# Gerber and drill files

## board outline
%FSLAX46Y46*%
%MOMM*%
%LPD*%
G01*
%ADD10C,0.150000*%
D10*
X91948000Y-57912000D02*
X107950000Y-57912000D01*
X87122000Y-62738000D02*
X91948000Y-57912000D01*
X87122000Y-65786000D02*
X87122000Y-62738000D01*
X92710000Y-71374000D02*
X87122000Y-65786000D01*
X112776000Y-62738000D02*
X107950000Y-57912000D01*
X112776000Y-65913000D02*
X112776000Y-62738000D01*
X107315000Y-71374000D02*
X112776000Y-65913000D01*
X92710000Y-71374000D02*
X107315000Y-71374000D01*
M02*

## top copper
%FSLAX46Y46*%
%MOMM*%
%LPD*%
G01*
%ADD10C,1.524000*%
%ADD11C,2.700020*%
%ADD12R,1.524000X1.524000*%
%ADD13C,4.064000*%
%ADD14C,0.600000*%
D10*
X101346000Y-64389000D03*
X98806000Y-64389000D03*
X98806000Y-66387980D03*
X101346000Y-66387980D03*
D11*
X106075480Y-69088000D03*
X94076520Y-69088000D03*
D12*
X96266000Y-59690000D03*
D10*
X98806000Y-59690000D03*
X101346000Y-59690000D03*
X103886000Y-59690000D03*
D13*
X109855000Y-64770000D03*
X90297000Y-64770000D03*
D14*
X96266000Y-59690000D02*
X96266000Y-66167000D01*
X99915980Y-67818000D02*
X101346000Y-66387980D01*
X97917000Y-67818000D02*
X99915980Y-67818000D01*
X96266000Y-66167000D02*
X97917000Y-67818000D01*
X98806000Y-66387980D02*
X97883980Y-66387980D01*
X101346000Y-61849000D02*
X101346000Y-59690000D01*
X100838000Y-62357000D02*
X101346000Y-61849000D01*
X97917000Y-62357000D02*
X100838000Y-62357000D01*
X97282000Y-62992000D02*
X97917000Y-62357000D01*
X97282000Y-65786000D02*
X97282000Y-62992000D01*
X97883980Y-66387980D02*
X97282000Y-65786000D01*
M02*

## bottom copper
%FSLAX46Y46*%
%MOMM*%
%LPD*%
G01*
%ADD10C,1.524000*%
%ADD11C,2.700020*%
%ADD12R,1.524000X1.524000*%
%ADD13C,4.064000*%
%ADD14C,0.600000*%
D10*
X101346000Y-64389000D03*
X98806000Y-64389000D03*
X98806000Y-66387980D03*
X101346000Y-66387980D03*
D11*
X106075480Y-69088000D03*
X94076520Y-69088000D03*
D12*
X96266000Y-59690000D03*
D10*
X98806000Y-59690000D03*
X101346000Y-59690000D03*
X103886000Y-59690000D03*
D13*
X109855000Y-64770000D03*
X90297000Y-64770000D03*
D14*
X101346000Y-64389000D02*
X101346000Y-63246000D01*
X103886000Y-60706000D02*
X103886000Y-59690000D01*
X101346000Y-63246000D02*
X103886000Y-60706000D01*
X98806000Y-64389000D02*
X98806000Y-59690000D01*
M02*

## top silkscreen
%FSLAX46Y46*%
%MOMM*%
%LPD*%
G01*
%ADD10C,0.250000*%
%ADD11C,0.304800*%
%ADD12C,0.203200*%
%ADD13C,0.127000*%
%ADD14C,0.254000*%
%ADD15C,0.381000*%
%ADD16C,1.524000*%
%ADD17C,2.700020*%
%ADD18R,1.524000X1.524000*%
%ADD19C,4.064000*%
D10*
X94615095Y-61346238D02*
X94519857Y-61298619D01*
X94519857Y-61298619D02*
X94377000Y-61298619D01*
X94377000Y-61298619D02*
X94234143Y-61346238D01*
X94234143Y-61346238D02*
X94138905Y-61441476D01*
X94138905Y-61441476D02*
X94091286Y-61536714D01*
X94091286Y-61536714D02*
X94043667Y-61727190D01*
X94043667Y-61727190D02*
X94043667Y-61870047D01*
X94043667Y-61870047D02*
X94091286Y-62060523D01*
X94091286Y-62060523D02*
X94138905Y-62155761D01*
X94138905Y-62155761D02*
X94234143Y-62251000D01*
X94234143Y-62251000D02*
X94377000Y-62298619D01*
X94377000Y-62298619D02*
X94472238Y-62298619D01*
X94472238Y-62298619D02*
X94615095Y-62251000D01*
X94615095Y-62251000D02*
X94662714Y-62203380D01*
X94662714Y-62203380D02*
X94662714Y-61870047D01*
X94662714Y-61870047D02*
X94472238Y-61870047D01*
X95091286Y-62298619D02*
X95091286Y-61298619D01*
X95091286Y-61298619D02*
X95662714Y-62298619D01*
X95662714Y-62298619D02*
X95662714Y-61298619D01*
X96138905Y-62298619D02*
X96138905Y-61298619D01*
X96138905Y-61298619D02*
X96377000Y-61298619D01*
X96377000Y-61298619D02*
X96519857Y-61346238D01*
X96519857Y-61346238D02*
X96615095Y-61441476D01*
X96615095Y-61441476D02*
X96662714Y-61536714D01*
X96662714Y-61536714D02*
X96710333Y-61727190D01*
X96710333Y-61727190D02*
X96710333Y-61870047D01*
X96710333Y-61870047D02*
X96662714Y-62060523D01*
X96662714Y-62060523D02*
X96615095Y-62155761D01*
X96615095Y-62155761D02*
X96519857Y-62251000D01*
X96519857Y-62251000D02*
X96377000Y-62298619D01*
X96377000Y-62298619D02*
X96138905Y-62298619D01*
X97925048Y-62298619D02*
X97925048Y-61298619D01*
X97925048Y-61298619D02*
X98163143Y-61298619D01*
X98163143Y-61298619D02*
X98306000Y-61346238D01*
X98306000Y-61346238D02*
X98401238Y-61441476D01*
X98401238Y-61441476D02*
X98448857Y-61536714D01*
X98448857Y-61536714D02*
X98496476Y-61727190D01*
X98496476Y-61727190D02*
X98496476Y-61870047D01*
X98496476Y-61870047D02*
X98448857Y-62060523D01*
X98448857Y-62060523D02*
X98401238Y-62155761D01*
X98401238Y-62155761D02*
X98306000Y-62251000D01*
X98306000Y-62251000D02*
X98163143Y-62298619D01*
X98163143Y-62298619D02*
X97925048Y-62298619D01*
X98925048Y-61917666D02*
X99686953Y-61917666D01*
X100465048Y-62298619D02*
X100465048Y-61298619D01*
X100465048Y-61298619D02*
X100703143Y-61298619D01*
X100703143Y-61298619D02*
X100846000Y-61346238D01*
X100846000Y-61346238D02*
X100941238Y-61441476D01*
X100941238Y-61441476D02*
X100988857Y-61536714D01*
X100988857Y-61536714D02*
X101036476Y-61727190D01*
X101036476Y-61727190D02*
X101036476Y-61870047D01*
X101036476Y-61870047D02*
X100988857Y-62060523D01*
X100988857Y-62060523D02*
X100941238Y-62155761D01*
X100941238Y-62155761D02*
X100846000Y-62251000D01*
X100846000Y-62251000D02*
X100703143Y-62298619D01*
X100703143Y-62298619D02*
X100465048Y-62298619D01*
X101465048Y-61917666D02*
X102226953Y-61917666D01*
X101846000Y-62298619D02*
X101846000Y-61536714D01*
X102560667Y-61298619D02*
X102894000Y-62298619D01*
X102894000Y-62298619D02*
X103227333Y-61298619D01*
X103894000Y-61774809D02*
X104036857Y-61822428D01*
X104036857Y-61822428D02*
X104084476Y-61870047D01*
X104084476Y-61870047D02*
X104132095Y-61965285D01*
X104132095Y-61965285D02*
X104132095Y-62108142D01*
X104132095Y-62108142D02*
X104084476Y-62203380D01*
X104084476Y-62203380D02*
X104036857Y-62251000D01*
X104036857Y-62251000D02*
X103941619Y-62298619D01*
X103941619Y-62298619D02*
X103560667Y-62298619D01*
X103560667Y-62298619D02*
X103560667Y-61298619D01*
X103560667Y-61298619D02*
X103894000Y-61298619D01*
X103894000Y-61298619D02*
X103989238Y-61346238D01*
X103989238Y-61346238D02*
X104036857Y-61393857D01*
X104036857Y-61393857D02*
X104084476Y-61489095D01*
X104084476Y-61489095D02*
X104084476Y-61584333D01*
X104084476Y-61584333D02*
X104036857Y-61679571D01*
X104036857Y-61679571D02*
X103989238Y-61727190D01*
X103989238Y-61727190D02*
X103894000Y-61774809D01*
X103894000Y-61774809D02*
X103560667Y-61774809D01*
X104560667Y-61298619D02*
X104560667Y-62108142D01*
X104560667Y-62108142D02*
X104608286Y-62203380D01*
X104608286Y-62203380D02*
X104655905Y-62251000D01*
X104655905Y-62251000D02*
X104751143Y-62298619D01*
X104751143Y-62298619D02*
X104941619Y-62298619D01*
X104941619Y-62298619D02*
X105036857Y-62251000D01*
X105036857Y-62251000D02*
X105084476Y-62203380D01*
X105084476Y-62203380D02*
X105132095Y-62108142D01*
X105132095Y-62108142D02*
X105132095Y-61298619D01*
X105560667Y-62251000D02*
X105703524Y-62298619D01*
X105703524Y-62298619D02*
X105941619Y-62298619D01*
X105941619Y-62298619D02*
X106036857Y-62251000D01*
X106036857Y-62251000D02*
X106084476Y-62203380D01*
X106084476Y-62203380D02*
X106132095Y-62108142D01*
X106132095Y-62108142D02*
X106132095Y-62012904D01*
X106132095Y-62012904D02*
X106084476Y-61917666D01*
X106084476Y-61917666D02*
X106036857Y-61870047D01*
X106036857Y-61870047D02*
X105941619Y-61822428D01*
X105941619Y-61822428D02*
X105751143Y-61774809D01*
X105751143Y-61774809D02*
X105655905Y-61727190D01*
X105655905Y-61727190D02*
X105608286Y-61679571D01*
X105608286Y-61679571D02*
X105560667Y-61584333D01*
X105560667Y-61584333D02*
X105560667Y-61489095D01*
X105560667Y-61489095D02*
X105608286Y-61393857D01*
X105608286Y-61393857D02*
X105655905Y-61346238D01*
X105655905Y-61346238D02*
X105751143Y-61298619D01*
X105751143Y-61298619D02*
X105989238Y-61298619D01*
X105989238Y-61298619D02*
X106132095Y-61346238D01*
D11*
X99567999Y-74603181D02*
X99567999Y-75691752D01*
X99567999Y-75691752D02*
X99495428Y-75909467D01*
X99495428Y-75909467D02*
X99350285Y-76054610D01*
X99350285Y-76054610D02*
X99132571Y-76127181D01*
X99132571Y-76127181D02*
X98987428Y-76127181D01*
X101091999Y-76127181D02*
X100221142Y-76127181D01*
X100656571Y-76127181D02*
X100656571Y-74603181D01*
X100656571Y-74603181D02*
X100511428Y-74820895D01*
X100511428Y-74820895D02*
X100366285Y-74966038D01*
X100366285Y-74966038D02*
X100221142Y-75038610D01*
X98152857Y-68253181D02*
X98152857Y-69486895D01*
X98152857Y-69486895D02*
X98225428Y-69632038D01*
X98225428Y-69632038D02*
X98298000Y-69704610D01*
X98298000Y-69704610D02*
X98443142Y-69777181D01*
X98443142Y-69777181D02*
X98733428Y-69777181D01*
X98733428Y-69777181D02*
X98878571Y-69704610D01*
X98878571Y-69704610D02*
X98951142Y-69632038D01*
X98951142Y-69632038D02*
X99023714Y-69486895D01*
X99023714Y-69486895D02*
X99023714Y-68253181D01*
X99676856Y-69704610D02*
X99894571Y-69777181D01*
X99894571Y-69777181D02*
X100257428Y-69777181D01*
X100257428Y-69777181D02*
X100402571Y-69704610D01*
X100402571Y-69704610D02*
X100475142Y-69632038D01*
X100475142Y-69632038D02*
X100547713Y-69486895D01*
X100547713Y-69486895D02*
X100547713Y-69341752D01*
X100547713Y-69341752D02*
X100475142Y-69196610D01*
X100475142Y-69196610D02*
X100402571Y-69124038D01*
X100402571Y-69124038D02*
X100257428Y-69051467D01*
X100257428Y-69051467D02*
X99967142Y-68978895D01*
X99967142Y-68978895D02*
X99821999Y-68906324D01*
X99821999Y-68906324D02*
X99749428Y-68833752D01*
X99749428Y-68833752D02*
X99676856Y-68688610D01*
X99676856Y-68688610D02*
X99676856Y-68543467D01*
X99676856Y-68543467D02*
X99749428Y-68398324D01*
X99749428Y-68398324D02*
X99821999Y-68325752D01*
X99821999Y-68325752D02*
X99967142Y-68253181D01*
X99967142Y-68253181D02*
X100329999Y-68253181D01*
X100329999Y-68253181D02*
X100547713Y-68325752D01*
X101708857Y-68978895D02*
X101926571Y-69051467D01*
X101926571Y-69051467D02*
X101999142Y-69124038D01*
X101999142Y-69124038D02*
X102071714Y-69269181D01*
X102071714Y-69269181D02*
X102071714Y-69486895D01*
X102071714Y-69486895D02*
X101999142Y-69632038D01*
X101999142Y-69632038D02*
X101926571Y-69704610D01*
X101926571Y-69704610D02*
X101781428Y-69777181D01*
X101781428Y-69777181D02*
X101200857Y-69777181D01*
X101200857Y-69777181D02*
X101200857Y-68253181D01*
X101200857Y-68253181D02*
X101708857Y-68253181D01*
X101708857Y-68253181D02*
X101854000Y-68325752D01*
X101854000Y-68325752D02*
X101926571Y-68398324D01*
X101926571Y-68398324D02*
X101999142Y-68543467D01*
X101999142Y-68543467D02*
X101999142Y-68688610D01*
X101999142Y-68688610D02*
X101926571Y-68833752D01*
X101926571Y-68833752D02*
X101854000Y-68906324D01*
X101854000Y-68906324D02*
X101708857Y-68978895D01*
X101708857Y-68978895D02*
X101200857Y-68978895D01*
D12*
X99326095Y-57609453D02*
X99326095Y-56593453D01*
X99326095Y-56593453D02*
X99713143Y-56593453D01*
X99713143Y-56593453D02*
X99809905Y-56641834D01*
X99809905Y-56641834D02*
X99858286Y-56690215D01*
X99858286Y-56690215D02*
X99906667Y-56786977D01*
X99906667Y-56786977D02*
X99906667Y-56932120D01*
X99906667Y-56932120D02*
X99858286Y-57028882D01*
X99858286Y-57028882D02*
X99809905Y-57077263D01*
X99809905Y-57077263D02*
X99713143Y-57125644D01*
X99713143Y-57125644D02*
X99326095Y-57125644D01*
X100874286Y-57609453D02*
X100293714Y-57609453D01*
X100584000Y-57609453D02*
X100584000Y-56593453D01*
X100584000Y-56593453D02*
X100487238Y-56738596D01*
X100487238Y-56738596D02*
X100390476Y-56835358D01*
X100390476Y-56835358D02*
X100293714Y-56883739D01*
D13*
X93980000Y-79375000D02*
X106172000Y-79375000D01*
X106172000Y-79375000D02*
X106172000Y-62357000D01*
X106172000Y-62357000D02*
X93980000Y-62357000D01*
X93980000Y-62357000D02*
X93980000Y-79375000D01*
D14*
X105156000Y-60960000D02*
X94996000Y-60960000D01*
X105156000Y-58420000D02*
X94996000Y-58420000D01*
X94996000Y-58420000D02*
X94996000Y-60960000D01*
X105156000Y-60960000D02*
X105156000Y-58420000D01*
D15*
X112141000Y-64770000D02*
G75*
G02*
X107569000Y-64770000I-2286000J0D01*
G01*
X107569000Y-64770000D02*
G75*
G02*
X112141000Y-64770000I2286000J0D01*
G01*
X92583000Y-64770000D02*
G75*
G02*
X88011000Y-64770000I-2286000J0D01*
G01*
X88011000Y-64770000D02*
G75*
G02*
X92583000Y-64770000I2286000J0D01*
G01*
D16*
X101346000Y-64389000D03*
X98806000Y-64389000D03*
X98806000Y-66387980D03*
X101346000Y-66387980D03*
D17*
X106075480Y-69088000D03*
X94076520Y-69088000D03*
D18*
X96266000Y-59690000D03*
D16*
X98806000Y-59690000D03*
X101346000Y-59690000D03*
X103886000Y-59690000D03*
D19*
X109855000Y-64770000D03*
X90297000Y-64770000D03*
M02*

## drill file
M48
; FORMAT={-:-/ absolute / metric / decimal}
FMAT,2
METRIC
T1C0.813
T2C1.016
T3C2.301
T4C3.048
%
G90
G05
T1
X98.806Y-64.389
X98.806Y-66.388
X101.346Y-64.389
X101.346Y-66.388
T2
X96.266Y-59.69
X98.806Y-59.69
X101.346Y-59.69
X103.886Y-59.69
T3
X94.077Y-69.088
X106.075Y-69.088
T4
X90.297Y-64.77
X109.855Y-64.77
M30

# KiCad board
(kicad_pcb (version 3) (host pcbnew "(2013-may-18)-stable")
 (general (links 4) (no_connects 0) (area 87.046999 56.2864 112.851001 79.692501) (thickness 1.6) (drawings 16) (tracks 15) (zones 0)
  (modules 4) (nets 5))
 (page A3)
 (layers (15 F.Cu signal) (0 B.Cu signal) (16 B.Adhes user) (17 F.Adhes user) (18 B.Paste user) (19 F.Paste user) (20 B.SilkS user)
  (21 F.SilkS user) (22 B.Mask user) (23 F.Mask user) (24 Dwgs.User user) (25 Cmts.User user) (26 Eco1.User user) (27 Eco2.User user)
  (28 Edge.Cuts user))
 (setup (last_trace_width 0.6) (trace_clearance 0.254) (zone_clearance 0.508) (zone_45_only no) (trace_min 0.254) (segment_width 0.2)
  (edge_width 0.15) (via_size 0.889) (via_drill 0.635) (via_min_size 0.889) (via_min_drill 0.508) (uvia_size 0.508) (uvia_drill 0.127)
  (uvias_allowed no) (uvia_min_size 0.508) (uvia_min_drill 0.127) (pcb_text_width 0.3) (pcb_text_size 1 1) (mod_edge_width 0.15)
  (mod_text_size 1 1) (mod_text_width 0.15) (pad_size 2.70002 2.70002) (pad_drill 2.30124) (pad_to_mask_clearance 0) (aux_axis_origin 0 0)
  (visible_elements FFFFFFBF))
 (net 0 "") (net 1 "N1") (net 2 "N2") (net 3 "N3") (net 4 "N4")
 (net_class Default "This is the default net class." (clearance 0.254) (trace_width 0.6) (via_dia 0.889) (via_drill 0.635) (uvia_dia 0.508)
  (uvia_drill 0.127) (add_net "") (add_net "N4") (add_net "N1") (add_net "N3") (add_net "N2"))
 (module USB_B (layer F.Cu) (at 100.076 69.088)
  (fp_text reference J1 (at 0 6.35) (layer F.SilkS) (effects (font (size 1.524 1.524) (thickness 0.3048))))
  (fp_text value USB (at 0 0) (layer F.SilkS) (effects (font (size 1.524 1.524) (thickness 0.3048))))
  (fp_line (start -6.096 10.287) (end 6.096 10.287) (layer F.SilkS) (width 0.127))
  (fp_line (start 6.096 10.287) (end 6.096 -6.731) (layer F.SilkS) (width 0.127))
  (fp_line (start 6.096 -6.731) (end -6.096 -6.731) (layer F.SilkS) (width 0.127))
  (fp_line (start -6.096 -6.731) (end -6.096 10.287) (layer F.SilkS) (width 0.127))
  (pad 1 thru_hole circle (at 1.27 -4.699) (size 1.524 1.524) (drill 0.8128) (layers *.Cu *.Mask F.SilkS) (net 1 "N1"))
  (pad 2 thru_hole circle (at -1.27 -4.699) (size 1.524 1.524) (drill 0.8128) (layers *.Cu *.Mask F.SilkS) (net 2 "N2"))
  (pad 3 thru_hole circle (at -1.27 -2.70002) (size 1.524 1.524) (drill 0.8128) (layers *.Cu *.Mask F.SilkS) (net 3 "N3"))
  (pad 4 thru_hole circle (at 1.27 -2.70002) (size 1.524 1.524) (drill 0.8128) (layers *.Cu *.Mask F.SilkS) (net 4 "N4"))
  (pad 5 thru_hole circle (at 5.99948 0) (size 2.70002 2.70002) (drill 2.30124) (layers *.Cu *.Mask F.SilkS))
  (pad 6 thru_hole circle (at -5.99948 0) (size 2.70002 2.70002) (drill 2.30124) (layers *.Cu *.Mask F.SilkS)))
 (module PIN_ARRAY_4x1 (layer F.Cu) (at 100.076 59.69)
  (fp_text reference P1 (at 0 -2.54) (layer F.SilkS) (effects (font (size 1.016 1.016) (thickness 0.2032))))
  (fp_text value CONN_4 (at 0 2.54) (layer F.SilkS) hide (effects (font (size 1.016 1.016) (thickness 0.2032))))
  (fp_line (start 5.08 1.27) (end -5.08 1.27) (layer F.SilkS) (width 0.254))
  (fp_line (start 5.08 -1.27) (end -5.08 -1.27) (layer F.SilkS) (width 0.254))
  (fp_line (start -5.08 -1.27) (end -5.08 1.27) (layer F.SilkS) (width 0.254))
  (fp_line (start 5.08 1.27) (end 5.08 -1.27) (layer F.SilkS) (width 0.254))
  (pad 1 thru_hole rect (at -3.81 0) (size 1.524 1.524) (drill 1.016) (layers *.Cu *.Mask F.SilkS) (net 4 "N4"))
  (pad 2 thru_hole circle (at -1.27 0) (size 1.524 1.524) (drill 1.016) (layers *.Cu *.Mask F.SilkS) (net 2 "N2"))
  (pad 3 thru_hole circle (at 1.27 0) (size 1.524 1.524) (drill 1.016) (layers *.Cu *.Mask F.SilkS) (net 3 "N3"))
  (pad 4 thru_hole circle (at 3.81 0) (size 1.524 1.524) (drill 1.016) (layers *.Cu *.Mask F.SilkS) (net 1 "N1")))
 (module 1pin (layer F.Cu) (at 109.855 64.77)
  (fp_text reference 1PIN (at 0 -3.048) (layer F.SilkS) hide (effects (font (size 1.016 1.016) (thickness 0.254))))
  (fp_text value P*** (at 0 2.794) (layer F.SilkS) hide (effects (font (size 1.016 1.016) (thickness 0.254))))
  (fp_circle (center 0 0) (end 0 -2.286) (layer F.SilkS) (width 0.381))
  (pad 1 thru_hole circle (at 0 0) (size 4.064 4.064) (drill 3.048) (layers *.Cu *.Mask F.SilkS)))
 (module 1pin (layer F.Cu) (at 90.297 64.77)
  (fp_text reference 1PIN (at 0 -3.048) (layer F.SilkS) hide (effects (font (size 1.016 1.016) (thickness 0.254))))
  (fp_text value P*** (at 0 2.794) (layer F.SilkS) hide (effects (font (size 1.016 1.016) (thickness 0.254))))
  (fp_circle (center 0 0) (end 0 -2.286) (layer F.SilkS) (width 0.381))
  (pad 1 thru_hole circle (at 0 0) (size 4.064 4.064) (drill 3.048) (layers *.Cu *.Mask F.SilkS)))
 (gr_line (start 91.948 57.912) (end 107.95 57.912) (angle 90) (layer Edge.Cuts) (width 0.15))
 (gr_line (start 87.122 62.738) (end 91.948 57.912) (angle 90) (layer Edge.Cuts) (width 0.15))
 (gr_line (start 87.122 65.786) (end 87.122 62.738) (angle 90) (layer Edge.Cuts) (width 0.15))
 (gr_line (start 92.71 71.374) (end 87.122 65.786) (angle 90) (layer Edge.Cuts) (width 0.15))
 (gr_line (start 112.776 62.738) (end 107.95 57.912) (angle 90) (layer Edge.Cuts) (width 0.15))
 (gr_line (start 112.776 65.913) (end 112.776 62.738) (angle 90) (layer Edge.Cuts) (width 0.15))
 (gr_line (start 107.315 71.374) (end 112.776 65.913) (angle 90) (layer Edge.Cuts) (width 0.15))
 (gr_line (start 92.71 71.374) (end 107.315 71.374) (angle 90) (layer Edge.Cuts) (width 0.15))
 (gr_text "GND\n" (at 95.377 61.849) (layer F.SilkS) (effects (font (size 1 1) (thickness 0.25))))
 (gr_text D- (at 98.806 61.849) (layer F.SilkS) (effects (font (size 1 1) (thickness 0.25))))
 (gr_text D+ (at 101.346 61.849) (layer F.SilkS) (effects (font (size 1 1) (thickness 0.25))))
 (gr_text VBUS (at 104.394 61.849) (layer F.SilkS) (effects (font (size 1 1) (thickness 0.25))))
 (segment (start 96.266 59.69) (end 96.266 66.167) (width 0.6) (layer F.Cu) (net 4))
 (segment (start 99.91598 67.818) (end 101.346 66.38798) (width 0.6) (layer F.Cu) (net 4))
 (segment (start 97.917 67.818) (end 99.91598 67.818) (width 0.6) (layer F.Cu) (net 4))
 (segment (start 96.266 66.167) (end 97.917 67.818) (width 0.6) (layer F.Cu) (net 4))
 (segment (start 101.346 64.389) (end 101.346 63.246) (width 0.6) (layer B.Cu) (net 1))
 (segment (start 103.886 60.706) (end 103.886 59.69) (width 0.6) (layer B.Cu) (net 1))
 (segment (start 101.346 63.246) (end 103.886 60.706) (width 0.6) (layer B.Cu) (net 1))
 (segment (start 98.806 66.38798) (end 97.88398 66.38798) (width 0.6) (layer F.Cu) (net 3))
 (segment (start 101.346 61.849) (end 101.346 59.69) (width 0.6) (layer F.Cu) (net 3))
 (segment (start 100.838 62.357) (end 101.346 61.849) (width 0.6) (layer F.Cu) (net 3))
 (segment (start 97.917 62.357) (end 100.838 62.357) (width 0.6) (layer F.Cu) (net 3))
 (segment (start 97.282 62.992) (end 97.917 62.357) (width 0.6) (layer F.Cu) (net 3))
 (segment (start 97.282 65.786) (end 97.282 62.992) (width 0.6) (layer F.Cu) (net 3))
 (segment (start 97.88398 66.38798) (end 97.282 65.786) (width 0.6) (layer F.Cu) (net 3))
 (segment (start 98.806 64.389) (end 98.806 59.69) (width 0.6) (layer B.Cu) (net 2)))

